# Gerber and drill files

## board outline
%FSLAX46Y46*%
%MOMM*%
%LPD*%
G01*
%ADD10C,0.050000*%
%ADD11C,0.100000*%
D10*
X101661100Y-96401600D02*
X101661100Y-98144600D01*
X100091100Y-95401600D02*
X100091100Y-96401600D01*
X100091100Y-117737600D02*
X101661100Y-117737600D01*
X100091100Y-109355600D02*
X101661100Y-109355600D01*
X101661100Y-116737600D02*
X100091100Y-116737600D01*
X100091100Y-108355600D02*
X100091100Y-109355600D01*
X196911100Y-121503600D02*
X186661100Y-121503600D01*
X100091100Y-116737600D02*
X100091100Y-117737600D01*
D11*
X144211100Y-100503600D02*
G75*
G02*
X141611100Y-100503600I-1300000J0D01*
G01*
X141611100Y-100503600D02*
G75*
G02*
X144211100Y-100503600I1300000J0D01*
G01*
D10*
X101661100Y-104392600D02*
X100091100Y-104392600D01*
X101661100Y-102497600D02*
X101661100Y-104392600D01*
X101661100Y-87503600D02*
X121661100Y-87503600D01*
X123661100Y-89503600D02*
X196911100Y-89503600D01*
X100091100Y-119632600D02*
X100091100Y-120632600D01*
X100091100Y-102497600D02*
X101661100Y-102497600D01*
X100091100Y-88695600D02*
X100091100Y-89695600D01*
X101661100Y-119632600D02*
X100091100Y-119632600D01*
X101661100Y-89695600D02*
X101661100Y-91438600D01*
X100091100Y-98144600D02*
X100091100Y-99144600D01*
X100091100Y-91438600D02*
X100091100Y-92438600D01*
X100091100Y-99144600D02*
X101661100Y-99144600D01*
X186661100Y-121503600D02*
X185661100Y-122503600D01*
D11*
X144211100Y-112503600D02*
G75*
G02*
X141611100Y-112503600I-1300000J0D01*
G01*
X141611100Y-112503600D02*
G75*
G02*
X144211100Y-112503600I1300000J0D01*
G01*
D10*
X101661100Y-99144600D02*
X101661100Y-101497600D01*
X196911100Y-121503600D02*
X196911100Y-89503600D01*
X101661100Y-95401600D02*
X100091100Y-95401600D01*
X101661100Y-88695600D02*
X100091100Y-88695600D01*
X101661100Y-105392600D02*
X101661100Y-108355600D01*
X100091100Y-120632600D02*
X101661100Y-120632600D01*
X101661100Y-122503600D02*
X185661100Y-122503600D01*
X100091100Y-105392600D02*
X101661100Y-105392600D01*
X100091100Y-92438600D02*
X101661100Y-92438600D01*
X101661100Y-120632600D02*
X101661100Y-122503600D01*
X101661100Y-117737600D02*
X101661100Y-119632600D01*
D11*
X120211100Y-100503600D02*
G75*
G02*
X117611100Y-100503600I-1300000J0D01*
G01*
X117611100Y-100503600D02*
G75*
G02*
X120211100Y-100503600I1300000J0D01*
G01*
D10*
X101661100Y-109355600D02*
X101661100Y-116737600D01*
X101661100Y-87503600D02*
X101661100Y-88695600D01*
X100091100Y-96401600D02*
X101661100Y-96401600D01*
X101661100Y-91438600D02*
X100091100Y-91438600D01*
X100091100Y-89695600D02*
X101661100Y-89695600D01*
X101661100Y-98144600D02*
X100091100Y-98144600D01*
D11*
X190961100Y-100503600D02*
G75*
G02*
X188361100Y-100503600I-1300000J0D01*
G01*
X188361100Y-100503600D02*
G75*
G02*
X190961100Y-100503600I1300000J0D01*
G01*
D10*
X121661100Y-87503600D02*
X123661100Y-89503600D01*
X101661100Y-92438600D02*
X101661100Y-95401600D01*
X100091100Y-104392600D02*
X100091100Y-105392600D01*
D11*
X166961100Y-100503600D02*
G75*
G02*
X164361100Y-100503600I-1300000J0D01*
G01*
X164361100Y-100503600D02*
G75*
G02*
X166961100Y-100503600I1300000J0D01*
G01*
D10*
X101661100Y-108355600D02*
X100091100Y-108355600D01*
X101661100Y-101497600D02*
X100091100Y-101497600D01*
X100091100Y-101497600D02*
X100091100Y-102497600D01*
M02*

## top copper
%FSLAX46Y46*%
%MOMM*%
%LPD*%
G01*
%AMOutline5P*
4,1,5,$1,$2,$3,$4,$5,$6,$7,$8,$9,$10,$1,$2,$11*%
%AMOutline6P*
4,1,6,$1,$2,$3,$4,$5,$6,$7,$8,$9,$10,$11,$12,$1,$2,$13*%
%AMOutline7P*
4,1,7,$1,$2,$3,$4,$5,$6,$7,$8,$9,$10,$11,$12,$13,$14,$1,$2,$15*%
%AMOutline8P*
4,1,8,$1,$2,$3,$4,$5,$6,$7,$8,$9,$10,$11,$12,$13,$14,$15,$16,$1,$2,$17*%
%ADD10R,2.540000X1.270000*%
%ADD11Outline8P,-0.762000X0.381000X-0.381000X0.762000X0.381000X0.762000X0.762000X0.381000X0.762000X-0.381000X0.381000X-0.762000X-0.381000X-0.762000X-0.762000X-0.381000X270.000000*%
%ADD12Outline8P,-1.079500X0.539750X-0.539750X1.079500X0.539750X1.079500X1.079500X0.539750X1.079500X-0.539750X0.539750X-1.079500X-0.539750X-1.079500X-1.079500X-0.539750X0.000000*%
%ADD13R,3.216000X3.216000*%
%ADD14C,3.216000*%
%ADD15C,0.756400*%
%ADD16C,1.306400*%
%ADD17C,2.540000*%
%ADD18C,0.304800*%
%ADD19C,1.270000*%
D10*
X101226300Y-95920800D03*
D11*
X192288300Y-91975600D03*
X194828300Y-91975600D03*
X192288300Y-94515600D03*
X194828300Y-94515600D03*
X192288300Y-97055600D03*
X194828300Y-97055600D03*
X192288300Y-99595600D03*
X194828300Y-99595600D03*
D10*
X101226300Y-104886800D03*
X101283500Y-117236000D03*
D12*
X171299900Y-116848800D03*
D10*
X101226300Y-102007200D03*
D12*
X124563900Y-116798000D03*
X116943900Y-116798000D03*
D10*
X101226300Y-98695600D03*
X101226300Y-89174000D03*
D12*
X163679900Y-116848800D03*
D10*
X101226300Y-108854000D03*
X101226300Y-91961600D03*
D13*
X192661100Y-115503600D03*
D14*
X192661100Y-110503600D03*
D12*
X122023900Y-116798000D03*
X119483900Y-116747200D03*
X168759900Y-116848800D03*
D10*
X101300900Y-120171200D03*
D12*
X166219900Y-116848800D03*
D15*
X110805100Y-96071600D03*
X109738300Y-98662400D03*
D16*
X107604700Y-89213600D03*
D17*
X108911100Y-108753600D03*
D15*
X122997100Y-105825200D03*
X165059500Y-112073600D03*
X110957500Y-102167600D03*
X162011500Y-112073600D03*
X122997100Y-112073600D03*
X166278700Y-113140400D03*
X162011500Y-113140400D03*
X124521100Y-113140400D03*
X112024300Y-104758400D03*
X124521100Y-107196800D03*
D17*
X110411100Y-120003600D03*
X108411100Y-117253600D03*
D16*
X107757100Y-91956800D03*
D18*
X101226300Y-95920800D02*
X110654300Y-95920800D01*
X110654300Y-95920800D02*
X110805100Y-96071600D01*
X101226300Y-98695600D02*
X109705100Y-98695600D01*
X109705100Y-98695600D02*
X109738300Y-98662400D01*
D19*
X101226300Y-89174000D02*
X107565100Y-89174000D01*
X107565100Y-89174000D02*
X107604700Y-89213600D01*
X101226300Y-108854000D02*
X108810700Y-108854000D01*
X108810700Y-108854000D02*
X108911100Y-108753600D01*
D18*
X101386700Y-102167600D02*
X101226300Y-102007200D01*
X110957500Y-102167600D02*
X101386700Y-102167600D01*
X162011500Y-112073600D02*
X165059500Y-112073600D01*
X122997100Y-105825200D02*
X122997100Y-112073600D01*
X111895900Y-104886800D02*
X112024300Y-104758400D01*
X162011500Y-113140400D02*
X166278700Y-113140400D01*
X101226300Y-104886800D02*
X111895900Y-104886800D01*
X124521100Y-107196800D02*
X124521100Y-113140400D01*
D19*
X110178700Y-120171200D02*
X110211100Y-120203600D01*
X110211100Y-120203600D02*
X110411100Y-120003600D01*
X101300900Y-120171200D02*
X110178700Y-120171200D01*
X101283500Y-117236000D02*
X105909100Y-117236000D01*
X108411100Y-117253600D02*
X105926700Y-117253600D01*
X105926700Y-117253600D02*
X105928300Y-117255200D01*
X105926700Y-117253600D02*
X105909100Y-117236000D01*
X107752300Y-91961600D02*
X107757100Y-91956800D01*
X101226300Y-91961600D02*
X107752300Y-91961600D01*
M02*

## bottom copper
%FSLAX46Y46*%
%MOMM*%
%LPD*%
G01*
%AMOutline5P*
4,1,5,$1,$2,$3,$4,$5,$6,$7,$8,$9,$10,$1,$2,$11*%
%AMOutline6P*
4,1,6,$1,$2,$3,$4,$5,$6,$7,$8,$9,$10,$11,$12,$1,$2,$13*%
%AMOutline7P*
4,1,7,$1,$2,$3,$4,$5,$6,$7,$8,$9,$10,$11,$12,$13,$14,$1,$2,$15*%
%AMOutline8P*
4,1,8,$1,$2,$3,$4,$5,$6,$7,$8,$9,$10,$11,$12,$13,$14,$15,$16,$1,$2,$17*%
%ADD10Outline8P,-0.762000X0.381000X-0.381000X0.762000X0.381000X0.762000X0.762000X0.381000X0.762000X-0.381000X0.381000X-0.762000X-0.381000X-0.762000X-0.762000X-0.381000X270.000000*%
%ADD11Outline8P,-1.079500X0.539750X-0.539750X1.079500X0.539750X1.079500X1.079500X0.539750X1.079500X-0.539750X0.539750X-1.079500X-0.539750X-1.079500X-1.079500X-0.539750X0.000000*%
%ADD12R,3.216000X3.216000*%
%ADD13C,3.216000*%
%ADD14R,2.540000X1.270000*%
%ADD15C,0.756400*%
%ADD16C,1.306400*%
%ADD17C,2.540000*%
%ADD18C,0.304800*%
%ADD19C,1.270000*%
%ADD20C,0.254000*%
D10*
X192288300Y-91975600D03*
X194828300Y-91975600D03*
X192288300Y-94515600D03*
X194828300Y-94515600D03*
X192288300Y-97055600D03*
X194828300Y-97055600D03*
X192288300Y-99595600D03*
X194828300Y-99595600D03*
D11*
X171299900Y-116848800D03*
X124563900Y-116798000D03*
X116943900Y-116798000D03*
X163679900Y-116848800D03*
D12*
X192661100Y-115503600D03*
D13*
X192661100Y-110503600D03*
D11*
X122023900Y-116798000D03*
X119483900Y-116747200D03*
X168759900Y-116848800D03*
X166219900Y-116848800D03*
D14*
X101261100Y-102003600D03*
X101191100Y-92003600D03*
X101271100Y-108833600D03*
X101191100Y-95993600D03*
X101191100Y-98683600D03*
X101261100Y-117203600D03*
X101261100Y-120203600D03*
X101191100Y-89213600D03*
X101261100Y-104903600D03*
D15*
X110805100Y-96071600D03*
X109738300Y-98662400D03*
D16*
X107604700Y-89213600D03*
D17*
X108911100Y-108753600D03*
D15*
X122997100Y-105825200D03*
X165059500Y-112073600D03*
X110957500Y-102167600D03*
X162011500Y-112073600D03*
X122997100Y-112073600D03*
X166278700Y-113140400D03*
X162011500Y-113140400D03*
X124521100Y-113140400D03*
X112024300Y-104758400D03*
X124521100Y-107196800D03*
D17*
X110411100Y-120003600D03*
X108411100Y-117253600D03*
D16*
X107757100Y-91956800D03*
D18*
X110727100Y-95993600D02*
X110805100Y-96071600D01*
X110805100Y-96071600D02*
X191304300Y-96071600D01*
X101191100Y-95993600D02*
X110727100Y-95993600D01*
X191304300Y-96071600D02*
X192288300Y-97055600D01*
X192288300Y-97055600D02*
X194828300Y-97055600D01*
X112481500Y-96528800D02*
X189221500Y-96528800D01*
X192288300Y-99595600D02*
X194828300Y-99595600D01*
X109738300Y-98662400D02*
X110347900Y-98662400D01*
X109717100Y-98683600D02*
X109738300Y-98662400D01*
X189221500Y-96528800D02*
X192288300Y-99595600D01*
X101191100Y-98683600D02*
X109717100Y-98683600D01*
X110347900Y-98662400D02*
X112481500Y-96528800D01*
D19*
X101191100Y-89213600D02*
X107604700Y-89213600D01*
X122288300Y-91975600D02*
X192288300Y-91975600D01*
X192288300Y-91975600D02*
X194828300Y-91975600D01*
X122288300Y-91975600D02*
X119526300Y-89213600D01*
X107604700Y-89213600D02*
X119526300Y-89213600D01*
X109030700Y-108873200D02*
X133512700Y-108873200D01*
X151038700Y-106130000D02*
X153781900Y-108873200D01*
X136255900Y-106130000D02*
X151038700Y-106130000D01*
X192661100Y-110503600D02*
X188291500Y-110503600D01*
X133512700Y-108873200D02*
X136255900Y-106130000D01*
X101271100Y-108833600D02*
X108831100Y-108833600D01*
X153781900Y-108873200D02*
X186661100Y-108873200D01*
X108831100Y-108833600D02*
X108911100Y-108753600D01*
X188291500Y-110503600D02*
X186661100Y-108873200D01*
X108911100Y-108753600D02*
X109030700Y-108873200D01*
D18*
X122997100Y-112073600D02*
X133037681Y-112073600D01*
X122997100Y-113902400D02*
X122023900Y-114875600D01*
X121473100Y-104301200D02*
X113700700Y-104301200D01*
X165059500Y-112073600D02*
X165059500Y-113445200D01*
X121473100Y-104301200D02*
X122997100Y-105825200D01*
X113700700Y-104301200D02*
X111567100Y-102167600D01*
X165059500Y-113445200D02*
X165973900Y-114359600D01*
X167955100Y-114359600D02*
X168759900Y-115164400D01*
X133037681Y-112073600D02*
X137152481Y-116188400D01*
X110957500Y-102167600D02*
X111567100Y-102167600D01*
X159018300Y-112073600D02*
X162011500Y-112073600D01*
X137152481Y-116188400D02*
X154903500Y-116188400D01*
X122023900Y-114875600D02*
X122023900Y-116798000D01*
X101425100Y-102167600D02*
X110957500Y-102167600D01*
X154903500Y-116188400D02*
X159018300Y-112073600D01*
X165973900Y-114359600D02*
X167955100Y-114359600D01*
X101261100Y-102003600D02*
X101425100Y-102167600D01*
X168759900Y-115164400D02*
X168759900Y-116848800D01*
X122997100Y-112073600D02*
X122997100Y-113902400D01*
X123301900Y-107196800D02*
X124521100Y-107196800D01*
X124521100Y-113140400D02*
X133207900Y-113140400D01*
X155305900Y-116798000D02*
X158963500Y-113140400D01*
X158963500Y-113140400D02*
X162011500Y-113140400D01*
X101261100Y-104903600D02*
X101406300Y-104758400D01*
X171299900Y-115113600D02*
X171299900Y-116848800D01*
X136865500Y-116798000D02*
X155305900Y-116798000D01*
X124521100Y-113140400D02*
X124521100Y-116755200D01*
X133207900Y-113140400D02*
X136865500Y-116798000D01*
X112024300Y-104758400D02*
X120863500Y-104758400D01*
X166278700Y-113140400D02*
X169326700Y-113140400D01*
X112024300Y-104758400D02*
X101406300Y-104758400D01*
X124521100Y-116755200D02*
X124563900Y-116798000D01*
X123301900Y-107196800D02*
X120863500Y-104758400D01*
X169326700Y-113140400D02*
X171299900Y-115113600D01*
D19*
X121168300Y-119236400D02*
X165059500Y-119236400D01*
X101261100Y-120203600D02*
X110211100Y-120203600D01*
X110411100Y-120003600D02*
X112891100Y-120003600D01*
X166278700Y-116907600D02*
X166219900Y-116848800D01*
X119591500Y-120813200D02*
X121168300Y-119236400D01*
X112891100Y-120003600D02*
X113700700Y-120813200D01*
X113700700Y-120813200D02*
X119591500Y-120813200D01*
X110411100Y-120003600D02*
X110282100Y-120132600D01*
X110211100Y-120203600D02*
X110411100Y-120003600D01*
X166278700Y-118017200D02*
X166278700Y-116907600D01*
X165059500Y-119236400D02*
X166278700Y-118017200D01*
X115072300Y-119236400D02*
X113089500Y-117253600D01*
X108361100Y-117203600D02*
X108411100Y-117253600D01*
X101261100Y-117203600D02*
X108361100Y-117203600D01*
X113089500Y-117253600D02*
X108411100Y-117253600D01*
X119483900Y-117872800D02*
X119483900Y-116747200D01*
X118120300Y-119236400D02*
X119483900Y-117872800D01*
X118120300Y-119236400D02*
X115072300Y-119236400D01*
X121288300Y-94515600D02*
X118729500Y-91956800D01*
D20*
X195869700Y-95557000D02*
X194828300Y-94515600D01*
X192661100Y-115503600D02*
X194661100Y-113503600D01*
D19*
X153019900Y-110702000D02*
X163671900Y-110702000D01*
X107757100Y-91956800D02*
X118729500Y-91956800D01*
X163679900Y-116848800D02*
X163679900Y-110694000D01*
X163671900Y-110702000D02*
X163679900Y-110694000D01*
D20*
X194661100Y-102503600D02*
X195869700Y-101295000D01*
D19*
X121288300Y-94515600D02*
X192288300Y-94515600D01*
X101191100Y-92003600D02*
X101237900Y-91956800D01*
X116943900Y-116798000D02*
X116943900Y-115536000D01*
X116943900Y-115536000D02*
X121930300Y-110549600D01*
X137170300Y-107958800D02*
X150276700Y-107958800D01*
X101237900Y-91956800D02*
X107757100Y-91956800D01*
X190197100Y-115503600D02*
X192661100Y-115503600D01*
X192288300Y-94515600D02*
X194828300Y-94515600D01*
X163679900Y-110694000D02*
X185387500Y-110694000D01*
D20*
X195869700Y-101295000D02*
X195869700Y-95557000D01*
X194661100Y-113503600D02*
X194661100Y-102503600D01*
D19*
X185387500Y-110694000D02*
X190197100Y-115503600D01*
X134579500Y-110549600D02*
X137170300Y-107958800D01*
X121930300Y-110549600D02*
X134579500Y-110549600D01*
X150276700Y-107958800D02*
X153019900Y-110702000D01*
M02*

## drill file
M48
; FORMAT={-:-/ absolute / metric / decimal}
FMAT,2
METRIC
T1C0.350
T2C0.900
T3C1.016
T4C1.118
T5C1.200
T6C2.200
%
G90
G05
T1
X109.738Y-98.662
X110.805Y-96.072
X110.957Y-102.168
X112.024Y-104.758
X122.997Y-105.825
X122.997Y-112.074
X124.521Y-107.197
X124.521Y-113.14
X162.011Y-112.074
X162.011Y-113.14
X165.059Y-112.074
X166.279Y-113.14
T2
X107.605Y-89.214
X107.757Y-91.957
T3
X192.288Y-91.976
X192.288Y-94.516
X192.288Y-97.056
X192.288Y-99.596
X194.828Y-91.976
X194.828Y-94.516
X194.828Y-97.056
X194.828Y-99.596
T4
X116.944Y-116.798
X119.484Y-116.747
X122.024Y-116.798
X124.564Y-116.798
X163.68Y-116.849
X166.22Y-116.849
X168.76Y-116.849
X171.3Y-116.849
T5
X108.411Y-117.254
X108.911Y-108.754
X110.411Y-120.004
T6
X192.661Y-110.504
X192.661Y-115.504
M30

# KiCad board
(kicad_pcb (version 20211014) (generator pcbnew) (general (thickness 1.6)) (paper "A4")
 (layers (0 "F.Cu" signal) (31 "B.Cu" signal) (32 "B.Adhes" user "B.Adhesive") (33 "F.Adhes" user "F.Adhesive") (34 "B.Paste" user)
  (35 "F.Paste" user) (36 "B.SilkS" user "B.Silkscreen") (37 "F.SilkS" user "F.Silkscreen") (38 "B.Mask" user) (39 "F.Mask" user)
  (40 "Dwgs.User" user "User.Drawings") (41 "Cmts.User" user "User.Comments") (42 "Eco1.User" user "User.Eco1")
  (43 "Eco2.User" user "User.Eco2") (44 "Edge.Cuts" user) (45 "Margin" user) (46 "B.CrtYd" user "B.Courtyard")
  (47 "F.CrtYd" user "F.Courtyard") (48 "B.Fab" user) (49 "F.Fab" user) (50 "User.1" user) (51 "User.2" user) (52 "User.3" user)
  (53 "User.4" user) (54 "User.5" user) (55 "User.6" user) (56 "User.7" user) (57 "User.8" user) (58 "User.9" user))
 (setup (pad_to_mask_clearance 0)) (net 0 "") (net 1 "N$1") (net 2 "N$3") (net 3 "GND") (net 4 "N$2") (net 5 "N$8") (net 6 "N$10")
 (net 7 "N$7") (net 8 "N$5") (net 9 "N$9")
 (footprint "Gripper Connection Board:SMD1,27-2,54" (layer "F.Cu") (at 101.2263 95.9208 90)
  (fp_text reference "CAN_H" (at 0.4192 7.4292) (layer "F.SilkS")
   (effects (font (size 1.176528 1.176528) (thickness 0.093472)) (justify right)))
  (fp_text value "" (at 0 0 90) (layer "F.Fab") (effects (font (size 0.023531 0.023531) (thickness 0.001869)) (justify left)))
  (pad "1" smd rect (at 0 0 90) (size 1.27 2.54) (layers "F.Cu" "F.Paste" "F.Mask") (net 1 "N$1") (solder_mask_margin 0.1016)))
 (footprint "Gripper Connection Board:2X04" (layer "F.Cu") (at 193.5583 95.7856 -90)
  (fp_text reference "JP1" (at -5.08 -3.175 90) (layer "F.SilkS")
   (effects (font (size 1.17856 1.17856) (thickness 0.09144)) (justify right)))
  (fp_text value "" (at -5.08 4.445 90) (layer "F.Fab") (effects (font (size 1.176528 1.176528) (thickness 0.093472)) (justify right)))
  (pad "1" thru_hole roundrect (at -3.81 1.27 270) (size 1.524 1.524) (drill 1.016) (layers *.Cu *.Mask) (roundrect_rratio 0.25)
   (chamfer_ratio 0.25) (chamfer top_left top_right bottom_left bottom_right) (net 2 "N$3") (solder_mask_margin 0.1016))
  (pad "2" thru_hole roundrect (at -3.81 -1.27 270) (size 1.524 1.524) (drill 1.016) (layers *.Cu *.Mask) (roundrect_rratio 0.25)
   (chamfer_ratio 0.25) (chamfer top_left top_right bottom_left bottom_right) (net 2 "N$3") (solder_mask_margin 0.1016))
  (pad "3" thru_hole roundrect (at -1.27 1.27 270) (size 1.524 1.524) (drill 1.016) (layers *.Cu *.Mask) (roundrect_rratio 0.25)
   (chamfer_ratio 0.25) (chamfer top_left top_right bottom_left bottom_right) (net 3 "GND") (solder_mask_margin 0.1016))
  (pad "4" thru_hole roundrect (at -1.27 -1.27 270) (size 1.524 1.524) (drill 1.016) (layers *.Cu *.Mask) (roundrect_rratio 0.25)
   (chamfer_ratio 0.25) (chamfer top_left top_right bottom_left bottom_right) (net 3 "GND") (solder_mask_margin 0.1016))
  (pad "5" thru_hole roundrect (at 1.27 1.27 270) (size 1.524 1.524) (drill 1.016) (layers *.Cu *.Mask) (roundrect_rratio 0.25)
   (chamfer_ratio 0.25) (chamfer top_left top_right bottom_left bottom_right) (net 1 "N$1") (solder_mask_margin 0.1016))
  (pad "6" thru_hole roundrect (at 1.27 -1.27 270) (size 1.524 1.524) (drill 1.016) (layers *.Cu *.Mask) (roundrect_rratio 0.25)
   (chamfer_ratio 0.25) (chamfer top_left top_right bottom_left bottom_right) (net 1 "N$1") (solder_mask_margin 0.1016))
  (pad "7" thru_hole roundrect (at 3.81 1.27 270) (size 1.524 1.524) (drill 1.016) (layers *.Cu *.Mask) (roundrect_rratio 0.25)
   (chamfer_ratio 0.25) (chamfer top_left top_right bottom_left bottom_right) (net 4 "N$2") (solder_mask_margin 0.1016))
  (pad "8" thru_hole roundrect (at 3.81 -1.27 270) (size 1.524 1.524) (drill 1.016) (layers *.Cu *.Mask) (roundrect_rratio 0.25)
   (chamfer_ratio 0.25) (chamfer top_left top_right bottom_left bottom_right) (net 4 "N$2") (solder_mask_margin 0.1016)))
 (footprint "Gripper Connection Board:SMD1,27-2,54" (layer "F.Cu") (at 101.2263 104.8868 90)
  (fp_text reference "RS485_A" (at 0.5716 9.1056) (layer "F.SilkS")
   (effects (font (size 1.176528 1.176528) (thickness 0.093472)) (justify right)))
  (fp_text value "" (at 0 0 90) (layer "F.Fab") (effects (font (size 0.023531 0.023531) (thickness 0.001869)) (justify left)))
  (pad "1" smd rect (at 0 0 90) (size 1.27 2.54) (layers "F.Cu" "F.Paste" "F.Mask") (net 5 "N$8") (solder_mask_margin 0.1016)))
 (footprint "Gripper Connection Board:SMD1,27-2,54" (layer "F.Cu") (at 101.2835 117.236 90)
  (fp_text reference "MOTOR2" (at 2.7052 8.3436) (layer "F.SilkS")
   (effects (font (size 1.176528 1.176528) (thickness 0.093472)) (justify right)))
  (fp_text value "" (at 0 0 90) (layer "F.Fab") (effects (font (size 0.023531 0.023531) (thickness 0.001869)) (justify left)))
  (pad "1" smd rect (at 0 0 90) (size 1.27 2.54) (layers "F.Cu" "F.Paste" "F.Mask") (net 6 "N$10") (solder_mask_margin 0.1016)))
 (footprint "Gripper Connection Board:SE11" (layer "F.Cu") (at 171.2999 116.8488)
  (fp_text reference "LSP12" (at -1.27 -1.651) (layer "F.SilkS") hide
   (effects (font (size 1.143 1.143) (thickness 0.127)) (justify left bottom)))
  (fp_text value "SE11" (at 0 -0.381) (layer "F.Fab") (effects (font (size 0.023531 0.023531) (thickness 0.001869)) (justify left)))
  (pad "MP" thru_hole roundrect (at 0 0) (size 2.159 2.159) (drill 1.1176) (layers *.Cu *.Mask) (roundrect_rratio 0.25) (chamfer_ratio 0.25)
   (chamfer top_left top_right bottom_left bottom_right) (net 5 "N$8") (solder_mask_margin 0.1016)))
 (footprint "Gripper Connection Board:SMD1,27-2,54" (layer "F.Cu") (at 101.2263 102.0072 90)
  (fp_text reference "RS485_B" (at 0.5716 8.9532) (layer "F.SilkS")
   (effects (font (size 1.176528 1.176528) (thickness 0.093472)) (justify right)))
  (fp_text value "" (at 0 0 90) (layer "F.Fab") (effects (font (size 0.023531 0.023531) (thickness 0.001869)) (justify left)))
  (pad "1" smd rect (at 0 0 90) (size 1.27 2.54) (layers "F.Cu" "F.Paste" "F.Mask") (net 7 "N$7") (solder_mask_margin 0.1016)))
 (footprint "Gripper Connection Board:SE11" (layer "F.Cu") (at 124.5639 116.798)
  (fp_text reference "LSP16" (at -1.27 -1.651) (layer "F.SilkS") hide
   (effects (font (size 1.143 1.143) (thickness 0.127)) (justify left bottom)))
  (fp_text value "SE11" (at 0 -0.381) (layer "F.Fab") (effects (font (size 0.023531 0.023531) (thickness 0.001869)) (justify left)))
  (pad "MP" thru_hole roundrect (at 0 0) (size 2.159 2.159) (drill 1.1176) (layers *.Cu *.Mask) (roundrect_rratio 0.25) (chamfer_ratio 0.25)
   (chamfer top_left top_right bottom_left bottom_right) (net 5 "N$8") (solder_mask_margin 0.1016)))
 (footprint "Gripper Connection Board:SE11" (layer "F.Cu") (at 116.9439 116.798)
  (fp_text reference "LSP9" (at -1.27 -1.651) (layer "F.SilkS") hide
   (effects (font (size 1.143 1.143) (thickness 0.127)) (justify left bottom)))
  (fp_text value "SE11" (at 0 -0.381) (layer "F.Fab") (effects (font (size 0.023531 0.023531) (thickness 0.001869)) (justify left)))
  (pad "MP" thru_hole roundrect (at 0 0) (size 2.159 2.159) (drill 1.1176) (layers *.Cu *.Mask) (roundrect_rratio 0.25) (chamfer_ratio 0.25)
   (chamfer top_left top_right bottom_left bottom_right) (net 3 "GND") (solder_mask_margin 0.1016)))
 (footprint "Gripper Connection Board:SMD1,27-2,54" (layer "F.Cu") (at 101.2263 98.6956 90)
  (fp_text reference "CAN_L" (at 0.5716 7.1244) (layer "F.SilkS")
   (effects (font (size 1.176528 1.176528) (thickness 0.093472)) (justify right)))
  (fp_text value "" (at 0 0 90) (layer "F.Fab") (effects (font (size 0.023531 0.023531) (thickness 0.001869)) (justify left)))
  (pad "1" smd rect (at 0 0 90) (size 1.27 2.54) (layers "F.Cu" "F.Paste" "F.Mask") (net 4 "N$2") (solder_mask_margin 0.1016)))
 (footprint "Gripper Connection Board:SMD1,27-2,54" (layer "F.Cu") (at 101.2263 89.174 90)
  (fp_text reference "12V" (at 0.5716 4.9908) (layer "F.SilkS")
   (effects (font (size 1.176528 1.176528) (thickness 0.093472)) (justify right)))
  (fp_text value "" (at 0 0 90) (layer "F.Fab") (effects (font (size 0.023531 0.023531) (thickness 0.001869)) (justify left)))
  (pad "1" smd rect (at 0 0 90) (size 1.27 2.54) (layers "F.Cu" "F.Paste" "F.Mask") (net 2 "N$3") (solder_mask_margin 0.1016)))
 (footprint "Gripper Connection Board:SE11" (layer "F.Cu") (at 163.6799 116.8488)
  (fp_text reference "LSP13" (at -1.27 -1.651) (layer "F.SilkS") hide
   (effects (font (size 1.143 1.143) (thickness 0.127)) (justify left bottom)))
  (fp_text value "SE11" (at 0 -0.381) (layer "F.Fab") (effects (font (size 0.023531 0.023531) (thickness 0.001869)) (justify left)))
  (pad "MP" thru_hole roundrect (at 0 0) (size 2.159 2.159) (drill 1.1176) (layers *.Cu *.Mask) (roundrect_rratio 0.25) (chamfer_ratio 0.25)
   (chamfer top_left top_right bottom_left bottom_right) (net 3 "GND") (solder_mask_margin 0.1016)))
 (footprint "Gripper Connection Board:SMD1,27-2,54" (layer "F.Cu") (at 101.2263 108.854 90)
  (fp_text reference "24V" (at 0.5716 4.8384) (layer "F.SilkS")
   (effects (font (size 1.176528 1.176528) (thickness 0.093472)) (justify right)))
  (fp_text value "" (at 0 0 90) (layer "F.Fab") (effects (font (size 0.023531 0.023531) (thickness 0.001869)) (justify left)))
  (pad "1" smd rect (at 0 0 90) (size 1.27 2.54) (layers "F.Cu" "F.Paste" "F.Mask") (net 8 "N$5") (solder_mask_margin 0.1016)))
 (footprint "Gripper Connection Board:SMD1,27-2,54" (layer "F.Cu") (at 101.2263 91.9616 90)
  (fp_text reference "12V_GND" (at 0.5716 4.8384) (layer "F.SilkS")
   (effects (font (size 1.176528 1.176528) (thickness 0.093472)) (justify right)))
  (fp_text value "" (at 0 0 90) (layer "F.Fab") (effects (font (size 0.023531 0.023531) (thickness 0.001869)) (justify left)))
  (pad "1" smd rect (at 0 0 90) (size 1.27 2.54) (layers "F.Cu" "F.Paste" "F.Mask") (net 3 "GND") (solder_mask_margin 0.1016)))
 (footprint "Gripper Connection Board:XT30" (layer "F.Cu") (at 192.6611 113.5036 90)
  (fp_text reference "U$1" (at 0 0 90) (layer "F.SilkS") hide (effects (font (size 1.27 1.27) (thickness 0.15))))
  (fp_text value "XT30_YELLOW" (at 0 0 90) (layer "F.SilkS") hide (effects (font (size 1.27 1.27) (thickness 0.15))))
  (pad "P$1" thru_hole rect (at -2 0 90) (size 3.216 3.216) (drill 2.2) (layers *.Cu *.Mask) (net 3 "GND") (solder_mask_margin 0.1016))
  (pad "P$2" thru_hole circle (at 3 0 90) (size 3.216 3.216) (drill 2.2) (layers *.Cu *.Mask) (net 8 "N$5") (solder_mask_margin 0.1016)))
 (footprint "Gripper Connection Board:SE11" (layer "F.Cu") (at 122.0239 116.798)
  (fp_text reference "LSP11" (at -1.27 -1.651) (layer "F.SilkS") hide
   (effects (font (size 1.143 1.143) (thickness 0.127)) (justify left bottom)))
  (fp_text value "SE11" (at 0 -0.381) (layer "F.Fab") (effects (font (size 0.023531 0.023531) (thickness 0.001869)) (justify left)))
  (pad "MP" thru_hole roundrect (at 0 0) (size 2.159 2.159) (drill 1.1176) (layers *.Cu *.Mask) (roundrect_rratio 0.25) (chamfer_ratio 0.25)
   (chamfer top_left top_right bottom_left bottom_right) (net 7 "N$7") (solder_mask_margin 0.1016)))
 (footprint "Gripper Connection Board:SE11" (layer "F.Cu") (at 119.4839 116.7472)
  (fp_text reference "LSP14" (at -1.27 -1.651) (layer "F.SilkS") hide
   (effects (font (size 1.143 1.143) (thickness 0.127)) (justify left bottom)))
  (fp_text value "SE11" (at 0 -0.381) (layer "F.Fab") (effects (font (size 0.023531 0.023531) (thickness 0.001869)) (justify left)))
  (pad "MP" thru_hole roundrect (at 0 0) (size 2.159 2.159) (drill 1.1176) (layers *.Cu *.Mask) (roundrect_rratio 0.25) (chamfer_ratio 0.25)
   (chamfer top_left top_right bottom_left bottom_right) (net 6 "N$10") (solder_mask_margin 0.1016)))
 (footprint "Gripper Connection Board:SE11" (layer "F.Cu") (at 168.7599 116.8488)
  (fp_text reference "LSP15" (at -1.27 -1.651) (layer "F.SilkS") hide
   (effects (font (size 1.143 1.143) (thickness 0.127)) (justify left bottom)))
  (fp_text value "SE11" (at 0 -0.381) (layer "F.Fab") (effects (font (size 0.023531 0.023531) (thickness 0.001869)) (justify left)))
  (pad "MP" thru_hole roundrect (at 0 0) (size 2.159 2.159) (drill 1.1176) (layers *.Cu *.Mask) (roundrect_rratio 0.25) (chamfer_ratio 0.25)
   (chamfer top_left top_right bottom_left bottom_right) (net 7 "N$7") (solder_mask_margin 0.1016)))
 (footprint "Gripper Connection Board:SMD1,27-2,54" (layer "F.Cu") (at 101.3009 120.1712 90)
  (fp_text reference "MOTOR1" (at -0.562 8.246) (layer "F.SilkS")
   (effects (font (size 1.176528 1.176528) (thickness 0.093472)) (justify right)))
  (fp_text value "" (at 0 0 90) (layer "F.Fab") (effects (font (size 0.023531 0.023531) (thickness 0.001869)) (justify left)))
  (pad "1" smd rect (at 0 0 90) (size 1.27 2.54) (layers "F.Cu" "F.Paste" "F.Mask") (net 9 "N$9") (solder_mask_margin 0.1016)))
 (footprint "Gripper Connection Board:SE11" (layer "F.Cu") (at 166.2199 116.8488)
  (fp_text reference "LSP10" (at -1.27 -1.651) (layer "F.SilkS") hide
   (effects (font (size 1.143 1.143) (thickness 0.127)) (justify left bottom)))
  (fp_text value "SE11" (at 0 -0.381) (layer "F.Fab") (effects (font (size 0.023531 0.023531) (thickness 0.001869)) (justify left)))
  (pad "MP" thru_hole roundrect (at 0 0) (size 2.159 2.159) (drill 1.1176) (layers *.Cu *.Mask) (roundrect_rratio 0.25) (chamfer_ratio 0.25)
   (chamfer top_left top_right bottom_left bottom_right) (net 9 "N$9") (solder_mask_margin 0.1016)))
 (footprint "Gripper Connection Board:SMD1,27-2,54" (layer "B.Cu") (at 101.2611 102.0036 -90)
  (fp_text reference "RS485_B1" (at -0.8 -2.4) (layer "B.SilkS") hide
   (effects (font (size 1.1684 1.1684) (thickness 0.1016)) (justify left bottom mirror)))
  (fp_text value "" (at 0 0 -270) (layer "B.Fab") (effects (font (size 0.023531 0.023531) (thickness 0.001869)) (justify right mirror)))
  (pad "1" smd rect (at 0 0 270) (size 1.27 2.54) (layers "B.Cu" "B.Paste" "B.Mask") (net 7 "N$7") (solder_mask_margin 0.1016)))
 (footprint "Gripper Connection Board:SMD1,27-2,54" (layer "B.Cu") (at 101.1911 92.0036 -90)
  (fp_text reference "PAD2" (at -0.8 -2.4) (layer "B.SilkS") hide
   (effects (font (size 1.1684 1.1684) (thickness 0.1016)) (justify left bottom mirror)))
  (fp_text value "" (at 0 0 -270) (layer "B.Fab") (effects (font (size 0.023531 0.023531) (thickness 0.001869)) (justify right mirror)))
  (pad "1" smd rect (at 0 0 270) (size 1.27 2.54) (layers "B.Cu" "B.Paste" "B.Mask") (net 3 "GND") (solder_mask_margin 0.1016)))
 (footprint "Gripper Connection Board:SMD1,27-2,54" (layer "B.Cu") (at 101.2711 108.8336 -90)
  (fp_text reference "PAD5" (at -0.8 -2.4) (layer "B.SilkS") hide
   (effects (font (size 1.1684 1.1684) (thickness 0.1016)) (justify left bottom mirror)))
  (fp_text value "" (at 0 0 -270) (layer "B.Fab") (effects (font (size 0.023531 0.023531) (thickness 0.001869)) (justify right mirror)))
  (pad "1" smd rect (at 0 0 270) (size 1.27 2.54) (layers "B.Cu" "B.Paste" "B.Mask") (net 8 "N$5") (solder_mask_margin 0.1016)))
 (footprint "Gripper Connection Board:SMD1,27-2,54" (layer "B.Cu") (at 101.1911 95.9936 -90)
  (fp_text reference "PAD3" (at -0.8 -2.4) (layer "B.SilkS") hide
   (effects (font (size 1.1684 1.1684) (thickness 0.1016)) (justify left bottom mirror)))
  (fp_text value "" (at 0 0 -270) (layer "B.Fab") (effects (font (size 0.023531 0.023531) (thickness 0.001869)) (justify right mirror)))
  (pad "1" smd rect (at 0 0 270) (size 1.27 2.54) (layers "B.Cu" "B.Paste" "B.Mask") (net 1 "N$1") (solder_mask_margin 0.1016)))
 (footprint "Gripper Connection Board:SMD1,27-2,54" (layer "B.Cu") (at 101.1911 98.6836 -90)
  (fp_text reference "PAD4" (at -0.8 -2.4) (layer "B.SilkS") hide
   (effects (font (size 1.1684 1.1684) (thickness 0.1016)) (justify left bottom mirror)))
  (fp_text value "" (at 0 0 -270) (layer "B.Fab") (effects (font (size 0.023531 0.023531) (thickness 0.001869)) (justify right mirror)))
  (pad "1" smd rect (at 0 0 270) (size 1.27 2.54) (layers "B.Cu" "B.Paste" "B.Mask") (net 4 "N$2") (solder_mask_margin 0.1016)))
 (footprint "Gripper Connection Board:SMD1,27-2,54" (layer "B.Cu") (at 101.2611 117.2036 -90)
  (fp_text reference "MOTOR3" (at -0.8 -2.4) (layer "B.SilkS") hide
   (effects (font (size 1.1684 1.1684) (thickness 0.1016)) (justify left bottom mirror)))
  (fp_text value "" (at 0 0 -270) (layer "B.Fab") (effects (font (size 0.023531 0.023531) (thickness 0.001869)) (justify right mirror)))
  (pad "1" smd rect (at 0 0 270) (size 1.27 2.54) (layers "B.Cu" "B.Paste" "B.Mask") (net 6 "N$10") (solder_mask_margin 0.1016)))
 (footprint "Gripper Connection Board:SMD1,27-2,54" (layer "B.Cu") (at 101.2611 120.2036 -90)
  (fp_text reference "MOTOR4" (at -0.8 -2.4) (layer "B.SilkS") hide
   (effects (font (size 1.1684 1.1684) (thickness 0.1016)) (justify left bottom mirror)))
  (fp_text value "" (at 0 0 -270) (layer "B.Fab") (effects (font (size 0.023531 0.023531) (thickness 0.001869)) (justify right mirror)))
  (pad "1" smd rect (at 0 0 270) (size 1.27 2.54) (layers "B.Cu" "B.Paste" "B.Mask") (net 9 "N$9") (solder_mask_margin 0.1016)))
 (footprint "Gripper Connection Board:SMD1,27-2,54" (layer "B.Cu") (at 101.1911 89.2136 -90)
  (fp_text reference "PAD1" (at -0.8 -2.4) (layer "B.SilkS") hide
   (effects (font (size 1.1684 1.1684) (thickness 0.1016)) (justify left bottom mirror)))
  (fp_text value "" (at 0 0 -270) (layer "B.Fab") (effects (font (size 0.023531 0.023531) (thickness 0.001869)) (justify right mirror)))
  (pad "1" smd rect (at 0 0 270) (size 1.27 2.54) (layers "B.Cu" "B.Paste" "B.Mask") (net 2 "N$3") (solder_mask_margin 0.1016)))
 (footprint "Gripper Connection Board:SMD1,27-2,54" (layer "B.Cu") (at 101.2611 104.9036 -90)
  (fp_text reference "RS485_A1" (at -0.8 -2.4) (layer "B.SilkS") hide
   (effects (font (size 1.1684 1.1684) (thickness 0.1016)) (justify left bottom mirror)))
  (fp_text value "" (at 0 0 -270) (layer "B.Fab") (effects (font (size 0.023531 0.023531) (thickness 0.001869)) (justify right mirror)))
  (pad "1" smd rect (at 0 0 270) (size 1.27 2.54) (layers "B.Cu" "B.Paste" "B.Mask") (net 5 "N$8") (solder_mask_margin 0.1016)))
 (gr_line (start 101.6611 96.4016) (end 101.6611 98.1446) (layer "Edge.Cuts") (width 0.05))
 (gr_line (start 100.0911 95.4016) (end 100.0911 96.4016) (layer "Edge.Cuts") (width 0.05))
 (gr_line (start 100.0911 117.7376) (end 101.6611 117.7376) (layer "Edge.Cuts") (width 0.05))
 (gr_line (start 100.0911 109.3556) (end 101.6611 109.3556) (layer "Edge.Cuts") (width 0.05))
 (gr_line (start 101.6611 116.7376) (end 100.0911 116.7376) (layer "Edge.Cuts") (width 0.05))
 (gr_line (start 100.0911 108.3556) (end 100.0911 109.3556) (layer "Edge.Cuts") (width 0.05))
 (gr_line (start 196.9111 121.5036) (end 186.6611 121.5036) (layer "Edge.Cuts") (width 0.05))
 (gr_line (start 100.0911 116.7376) (end 100.0911 117.7376) (layer "Edge.Cuts") (width 0.05))
 (gr_circle (center 142.9111 100.5036) (end 144.2111 100.5036) (layer "Edge.Cuts") (width 0) (fill none))
 (gr_line (start 101.6611 104.3926) (end 100.0911 104.3926) (layer "Edge.Cuts") (width 0.05))
 (gr_line (start 101.6611 102.4976) (end 101.6611 104.3926) (layer "Edge.Cuts") (width 0.05))
 (gr_line (start 101.6611 87.5036) (end 121.6611 87.5036) (layer "Edge.Cuts") (width 0.05))
 (gr_line (start 123.6611 89.5036) (end 196.9111 89.5036) (layer "Edge.Cuts") (width 0.05))
 (gr_line (start 100.0911 119.6326) (end 100.0911 120.6326) (layer "Edge.Cuts") (width 0.05))
 (gr_line (start 100.0911 102.4976) (end 101.6611 102.4976) (layer "Edge.Cuts") (width 0.05))
 (gr_line (start 100.0911 88.6956) (end 100.0911 89.6956) (layer "Edge.Cuts") (width 0.05))
 (gr_line (start 101.6611 119.6326) (end 100.0911 119.6326) (layer "Edge.Cuts") (width 0.05))
 (gr_line (start 101.6611 89.6956) (end 101.6611 91.4386) (layer "Edge.Cuts") (width 0.05))
 (gr_line (start 100.0911 98.1446) (end 100.0911 99.1446) (layer "Edge.Cuts") (width 0.05))
 (gr_line (start 100.0911 91.4386) (end 100.0911 92.4386) (layer "Edge.Cuts") (width 0.05))
 (gr_line (start 100.0911 99.1446) (end 101.6611 99.1446) (layer "Edge.Cuts") (width 0.05))
 (gr_line (start 186.6611 121.5036) (end 185.6611 122.5036) (layer "Edge.Cuts") (width 0.05))
 (gr_circle (center 142.9111 112.5036) (end 144.2111 112.5036) (layer "Edge.Cuts") (width 0) (fill none))
 (gr_line (start 101.6611 99.1446) (end 101.6611 101.4976) (layer "Edge.Cuts") (width 0.05))
 (gr_line (start 196.9111 121.5036) (end 196.9111 89.5036) (layer "Edge.Cuts") (width 0.05))
 (gr_line (start 101.6611 95.4016) (end 100.0911 95.4016) (layer "Edge.Cuts") (width 0.05))
 (gr_line (start 101.6611 88.6956) (end 100.0911 88.6956) (layer "Edge.Cuts") (width 0.05))
 (gr_line (start 101.6611 105.3926) (end 101.6611 108.3556) (layer "Edge.Cuts") (width 0.05))
 (gr_line (start 100.0911 120.6326) (end 101.6611 120.6326) (layer "Edge.Cuts") (width 0.05))
 (gr_line (start 101.6611 122.5036) (end 185.6611 122.5036) (layer "Edge.Cuts") (width 0.05))
 (gr_line (start 100.0911 105.3926) (end 101.6611 105.3926) (layer "Edge.Cuts") (width 0.05))
 (gr_line (start 100.0911 92.4386) (end 101.6611 92.4386) (layer "Edge.Cuts") (width 0.05))
 (gr_line (start 101.6611 120.6326) (end 101.6611 122.5036) (layer "Edge.Cuts") (width 0.05))
 (gr_line (start 101.6611 117.7376) (end 101.6611 119.6326) (layer "Edge.Cuts") (width 0.05))
 (gr_circle (center 118.9111 100.5036) (end 120.2111 100.5036) (layer "Edge.Cuts") (width 0) (fill none))
 (gr_line (start 101.6611 109.3556) (end 101.6611 116.7376) (layer "Edge.Cuts") (width 0.05))
 (gr_line (start 101.6611 87.5036) (end 101.6611 88.6956) (layer "Edge.Cuts") (width 0.05))
 (gr_line (start 100.0911 96.4016) (end 101.6611 96.4016) (layer "Edge.Cuts") (width 0.05))
 (gr_line (start 101.6611 91.4386) (end 100.0911 91.4386) (layer "Edge.Cuts") (width 0.05))
 (gr_line (start 100.0911 89.6956) (end 101.6611 89.6956) (layer "Edge.Cuts") (width 0.05))
 (gr_line (start 101.6611 98.1446) (end 100.0911 98.1446) (layer "Edge.Cuts") (width 0.05))
 (gr_circle (center 189.6611 100.5036) (end 190.9611 100.5036) (layer "Edge.Cuts") (width 0) (fill none))
 (gr_line (start 121.6611 87.5036) (end 123.6611 89.5036) (layer "Edge.Cuts") (width 0.05))
 (gr_line (start 101.6611 92.4386) (end 101.6611 95.4016) (layer "Edge.Cuts") (width 0.05))
 (gr_line (start 100.0911 104.3926) (end 100.0911 105.3926) (layer "Edge.Cuts") (width 0.05))
 (gr_circle (center 165.6611 100.5036) (end 166.9611 100.5036) (layer "Edge.Cuts") (width 0) (fill none))
 (gr_line (start 101.6611 108.3556) (end 100.0911 108.3556) (layer "Edge.Cuts") (width 0.05))
 (gr_line (start 101.6611 101.4976) (end 100.0911 101.4976) (layer "Edge.Cuts") (width 0.05))
 (gr_line (start 100.0911 101.4976) (end 100.0911 102.4976) (layer "Edge.Cuts") (width 0.05))
 (segment (start 101.2263 95.9208) (end 110.6543 95.9208) (width 0.3048) (layer "F.Cu") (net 1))
 (segment (start 110.6543 95.9208) (end 110.8051 96.0716) (width 0.3048) (layer "F.Cu") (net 1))
 (via (at 110.8051 96.0716) (size 0.7564) (drill 0.35) (layers "F.Cu" "B.Cu") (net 1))
 (segment (start 110.7271 95.9936) (end 110.8051 96.0716) (width 0.3048) (layer "B.Cu") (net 1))
 (segment (start 110.8051 96.0716) (end 191.3043 96.0716) (width 0.3048) (layer "B.Cu") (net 1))
 (segment (start 101.1911 95.9936) (end 110.7271 95.9936) (width 0.3048) (layer "B.Cu") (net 1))
 (segment (start 191.3043 96.0716) (end 192.2883 97.0556) (width 0.3048) (layer "B.Cu") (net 1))
 (segment (start 192.2883 97.0556) (end 194.8283 97.0556) (width 0.3048) (layer "B.Cu") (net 1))
 (segment (start 101.2263 98.6956) (end 109.7051 98.6956) (width 0.3048) (layer "F.Cu") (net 4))
 (segment (start 109.7051 98.6956) (end 109.7383 98.6624) (width 0.3048) (layer "F.Cu") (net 4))
 (via (at 109.7383 98.6624) (size 0.7564) (drill 0.35) (layers "F.Cu" "B.Cu") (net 4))
 (segment (start 112.4815 96.5288) (end 189.2215 96.5288) (width 0.3048) (layer "B.Cu") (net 4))
 (segment (start 192.2883 99.5956) (end 194.8283 99.5956) (width 0.3048) (layer "B.Cu") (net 4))
 (segment (start 109.7383 98.6624) (end 110.3479 98.6624) (width 0.3048) (layer "B.Cu") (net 4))
 (segment (start 109.7171 98.6836) (end 109.7383 98.6624) (width 0.3048) (layer "B.Cu") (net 4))
 (segment (start 189.2215 96.5288) (end 192.2883 99.5956) (width 0.3048) (layer "B.Cu") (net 4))
 (segment (start 101.1911 98.6836) (end 109.7171 98.6836) (width 0.3048) (layer "B.Cu") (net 4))
 (segment (start 110.3479 98.6624) (end 112.4815 96.5288) (width 0.3048) (layer "B.Cu") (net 4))
 (segment (start 101.2263 89.174) (end 107.5651 89.174) (width 1.27) (layer "F.Cu") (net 2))
 (segment (start 107.5651 89.174) (end 107.6047 89.2136) (width 1.27) (layer "F.Cu") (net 2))
 (via (at 107.6047 89.2136) (size 1.3064) (drill 0.9) (layers "F.Cu" "B.Cu") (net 2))
 (segment (start 101.1911 89.2136) (end 107.6047 89.2136) (width 1.27) (layer "B.Cu") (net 2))
 (segment (start 122.2883 91.9756) (end 192.2883 91.9756) (width 1.27) (layer "B.Cu") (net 2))
 (segment (start 192.2883 91.9756) (end 194.8283 91.9756) (width 1.27) (layer "B.Cu") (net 2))
 (segment (start 122.2883 91.9756) (end 119.5263 89.2136) (width 1.27) (layer "B.Cu") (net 2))
 (segment (start 107.6047 89.2136) (end 119.5263 89.2136) (width 1.27) (layer "B.Cu") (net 2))
 (segment (start 101.2263 108.854) (end 108.8107 108.854) (width 1.27) (layer "F.Cu") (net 8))
 (segment (start 108.8107 108.854) (end 108.9111 108.7536) (width 1.27) (layer "F.Cu") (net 8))
 (via (at 108.9111 108.7536) (size 2.54) (drill 1.2) (layers "F.Cu" "B.Cu") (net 8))
 (segment (start 109.0307 108.8732) (end 133.5127 108.8732) (width 1.27) (layer "B.Cu") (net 8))
 (segment (start 151.0387 106.13) (end 153.7819 108.8732) (width 1.27) (layer "B.Cu") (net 8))
 (segment (start 136.2559 106.13) (end 151.0387 106.13) (width 1.27) (layer "B.Cu") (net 8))
 (segment (start 192.6611 110.5036) (end 188.2915 110.5036) (width 1.27) (layer "B.Cu") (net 8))
 (segment (start 133.5127 108.8732) (end 136.2559 106.13) (width 1.27) (layer "B.Cu") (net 8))
 (segment (start 101.2711 108.8336) (end 108.8311 108.8336) (width 1.27) (layer "B.Cu") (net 8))
 (segment (start 153.7819 108.8732) (end 186.6611 108.8732) (width 1.27) (layer "B.Cu") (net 8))
 (segment (start 108.8311 108.8336) (end 108.9111 108.7536) (width 1.27) (layer "B.Cu") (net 8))
 (segment (start 188.2915 110.5036) (end 186.6611 108.8732) (width 1.27) (layer "B.Cu") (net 8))
 (segment (start 108.9111 108.7536) (end 109.0307 108.8732) (width 1.27) (layer "B.Cu") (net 8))
 (segment (start 101.3867 102.1676) (end 101.2263 102.0072) (width 0.3048) (layer "F.Cu") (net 7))
 (segment (start 110.9575 102.1676) (end 101.3867 102.1676) (width 0.3048) (layer "F.Cu") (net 7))
 (segment (start 162.0115 112.0736) (end 165.0595 112.0736) (width 0.3048) (layer "F.Cu") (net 7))
 (segment (start 122.9971 105.8252) (end 122.9971 112.0736) (width 0.3048) (layer "F.Cu") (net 7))
 (via (at 122.9971 105.8252) (size 0.7564) (drill 0.35) (layers "F.Cu" "B.Cu") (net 7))
 (via (at 165.0595 112.0736) (size 0.7564) (drill 0.35) (layers "F.Cu" "B.Cu") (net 7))
 (via (at 110.9575 102.1676) (size 0.7564) (drill 0.35) (layers "F.Cu" "B.Cu") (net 7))
 (via (at 162.0115 112.0736) (size 0.7564) (drill 0.35) (layers "F.Cu" "B.Cu") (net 7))
 (via (at 122.9971 112.0736) (size 0.7564) (drill 0.35) (layers "F.Cu" "B.Cu") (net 7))
 (segment (start 122.9971 112.0736) (end 133.037681 112.0736) (width 0.3048) (layer "B.Cu") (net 7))
 (segment (start 122.9971 113.9024) (end 122.0239 114.8756) (width 0.3048) (layer "B.Cu") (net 7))
 (segment (start 121.4731 104.3012) (end 113.7007 104.3012) (width 0.3048) (layer "B.Cu") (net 7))
 (segment (start 165.0595 112.0736) (end 165.0595 113.4452) (width 0.3048) (layer "B.Cu") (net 7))
 (segment (start 121.4731 104.3012) (end 122.9971 105.8252) (width 0.3048) (layer "B.Cu") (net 7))
 (segment (start 113.7007 104.3012) (end 111.5671 102.1676) (width 0.3048) (layer "B.Cu") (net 7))
 (segment (start 165.0595 113.4452) (end 165.9739 114.3596) (width 0.3048) (layer "B.Cu") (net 7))
 (segment (start 167.9551 114.3596) (end 168.7599 115.1644) (width 0.3048) (layer "B.Cu") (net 7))
 (segment (start 133.037681 112.0736) (end 137.152481 116.1884) (width 0.3048) (layer "B.Cu") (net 7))
 (segment (start 110.9575 102.1676) (end 111.5671 102.1676) (width 0.3048) (layer "B.Cu") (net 7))
 (segment (start 159.0183 112.0736) (end 162.0115 112.0736) (width 0.3048) (layer "B.Cu") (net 7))
 (segment (start 137.152481 116.1884) (end 154.9035 116.1884) (width 0.3048) (layer "B.Cu") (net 7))
 (segment (start 122.0239 114.8756) (end 122.0239 116.798) (width 0.3048) (layer "B.Cu") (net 7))
 (segment (start 101.4251 102.1676) (end 110.9575 102.1676) (width 0.3048) (layer "B.Cu") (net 7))
 (segment (start 154.9035 116.1884) (end 159.0183 112.0736) (width 0.3048) (layer "B.Cu") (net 7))
 (segment (start 165.9739 114.3596) (end 167.9551 114.3596) (width 0.3048) (layer "B.Cu") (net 7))
 (segment (start 101.2611 102.0036) (end 101.4251 102.1676) (width 0.3048) (layer "B.Cu") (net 7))
 (segment (start 168.7599 115.1644) (end 168.7599 116.8488) (width 0.3048) (layer "B.Cu") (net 7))
 (segment (start 122.9971 112.0736) (end 122.9971 113.9024) (width 0.3048) (layer "B.Cu") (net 7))
 (segment (start 111.8959 104.8868) (end 112.0243 104.7584) (width 0.3048) (layer "F.Cu") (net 5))
 (segment (start 162.0115 113.1404) (end 166.2787 113.1404) (width 0.3048) (layer "F.Cu") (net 5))
 (segment (start 101.2263 104.8868) (end 111.8959 104.8868) (width 0.3048) (layer "F.Cu") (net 5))
 (segment (start 124.5211 107.1968) (end 124.5211 113.1404) (width 0.3048) (layer "F.Cu") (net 5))
 (via (at 166.2787 113.1404) (size 0.7564) (drill 0.35) (layers "F.Cu" "B.Cu") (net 5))
 (via (at 162.0115 113.1404) (size 0.7564) (drill 0.35) (layers "F.Cu" "B.Cu") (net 5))
 (via (at 124.5211 113.1404) (size 0.7564) (drill 0.35) (layers "F.Cu" "B.Cu") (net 5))
 (via (at 112.0243 104.7584) (size 0.7564) (drill 0.35) (layers "F.Cu" "B.Cu") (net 5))
 (via (at 124.5211 107.1968) (size 0.7564) (drill 0.35) (layers "F.Cu" "B.Cu") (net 5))
 (segment (start 123.3019 107.1968) (end 124.5211 107.1968) (width 0.3048) (layer "B.Cu") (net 5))
 (segment (start 124.5211 113.1404) (end 133.2079 113.1404) (width 0.3048) (layer "B.Cu") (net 5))
 (segment (start 155.3059 116.798) (end 158.9635 113.1404) (width 0.3048) (layer "B.Cu") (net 5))
 (segment (start 158.9635 113.1404) (end 162.0115 113.1404) (width 0.3048) (layer "B.Cu") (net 5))
 (segment (start 101.2611 104.9036) (end 101.4063 104.7584) (width 0.3048) (layer "B.Cu") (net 5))
 (segment (start 171.2999 115.1136) (end 171.2999 116.8488) (width 0.3048) (layer "B.Cu") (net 5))
 (segment (start 136.8655 116.798) (end 155.3059 116.798) (width 0.3048) (layer "B.Cu") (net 5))
 (segment (start 124.5211 113.1404) (end 124.5211 116.7552) (width 0.3048) (layer "B.Cu") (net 5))
 (segment (start 133.2079 113.1404) (end 136.8655 116.798) (width 0.3048) (layer "B.Cu") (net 5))
 (segment (start 112.0243 104.7584) (end 120.8635 104.7584) (width 0.3048) (layer "B.Cu") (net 5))
 (segment (start 166.2787 113.1404) (end 169.3267 113.1404) (width 0.3048) (layer "B.Cu") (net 5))
 (segment (start 112.0243 104.7584) (end 101.4063 104.7584) (width 0.3048) (layer "B.Cu") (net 5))
 (segment (start 124.5211 116.7552) (end 124.5639 116.798) (width 0.3048) (layer "B.Cu") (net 5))
 (segment (start 123.3019 107.1968) (end 120.8635 104.7584) (width 0.3048) (layer "B.Cu") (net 5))
 (segment (start 169.3267 113.1404) (end 171.2999 115.1136) (width 0.3048) (layer "B.Cu") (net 5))
 (segment (start 110.1787 120.1712) (end 110.2111 120.2036) (width 1.27) (layer "F.Cu") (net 9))
 (segment (start 110.2111 120.2036) (end 110.4111 120.0036) (width 1.27) (layer "F.Cu") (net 9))
 (segment (start 101.3009 120.1712) (end 110.1787 120.1712) (width 1.27) (layer "F.Cu") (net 9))
 (via (at 110.4111 120.0036) (size 2.54) (drill 1.2) (layers "F.Cu" "B.Cu") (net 9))
 (segment (start 121.1683 119.2364) (end 165.0595 119.2364) (width 1.27) (layer "B.Cu") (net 9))
 (segment (start 101.2611 120.2036) (end 110.2111 120.2036) (width 1.27) (layer "B.Cu") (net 9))
 (segment (start 110.4111 120.0036) (end 112.8911 120.0036) (width 1.27) (layer "B.Cu") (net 9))
 (segment (start 166.2787 116.9076) (end 166.2199 116.8488) (width 1.27) (layer "B.Cu") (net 9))
 (segment (start 119.5915 120.8132) (end 121.1683 119.2364) (width 1.27) (layer "B.Cu") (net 9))
 (segment (start 112.8911 120.0036) (end 113.7007 120.8132) (width 1.27) (layer "B.Cu") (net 9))
 (segment (start 113.7007 120.8132) (end 119.5915 120.8132) (width 1.27) (layer "B.Cu") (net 9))
 (segment (start 110.4111 120.0036) (end 110.2821 120.1326) (width 1.27) (layer "B.Cu") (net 9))
 (segment (start 110.2111 120.2036) (end 110.4111 120.0036) (width 1.27) (layer "B.Cu") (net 9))
 (segment (start 166.2787 118.0172) (end 166.2787 116.9076) (width 1.27) (layer "B.Cu") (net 9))
 (segment (start 165.0595 119.2364) (end 166.2787 118.0172) (width 1.27) (layer "B.Cu") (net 9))
 (segment (start 101.2835 117.236) (end 105.9091 117.236) (width 1.27) (layer "F.Cu") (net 6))
 (segment (start 108.4111 117.2536) (end 105.9267 117.2536) (width 1.27) (layer "F.Cu") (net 6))
 (segment (start 105.9267 117.2536) (end 105.9283 117.2552) (width 1.27) (layer "F.Cu") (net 6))
 (segment (start 105.9267 117.2536) (end 105.9091 117.236) (width 1.27) (layer "F.Cu") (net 6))
 (via (at 108.4111 117.2536) (size 2.54) (drill 1.2) (layers "F.Cu" "B.Cu") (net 6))
 (segment (start 115.0723 119.2364) (end 113.0895 117.2536) (width 1.27) (layer "B.Cu") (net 6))
 (segment (start 108.3611 117.2036) (end 108.4111 117.2536) (width 1.27) (layer "B.Cu") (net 6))
 (segment (start 101.2611 117.2036) (end 108.3611 117.2036) (width 1.27) (layer "B.Cu") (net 6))
 (segment (start 113.0895 117.2536) (end 108.4111 117.2536) (width 1.27) (layer "B.Cu") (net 6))
 (segment (start 119.4839 117.8728) (end 119.4839 116.7472) (width 1.27) (layer "B.Cu") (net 6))
 (segment (start 118.1203 119.2364) (end 119.4839 117.8728) (width 1.27) (layer "B.Cu") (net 6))
 (segment (start 118.1203 119.2364) (end 115.0723 119.2364) (width 1.27) (layer "B.Cu") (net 6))
 (segment (start 107.7523 91.9616) (end 107.7571 91.9568) (width 1.27) (layer "F.Cu") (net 3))
 (segment (start 101.2263 91.9616) (end 107.7523 91.9616) (width 1.27) (layer "F.Cu") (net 3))
 (via (at 107.7571 91.9568) (size 1.3064) (drill 0.9) (layers "F.Cu" "B.Cu") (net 3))
 (segment (start 121.2883 94.5156) (end 118.7295 91.9568) (width 1.27) (layer "B.Cu") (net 3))
 (segment (start 195.8697 95.557) (end 194.8283 94.5156) (width 0.254) (layer "B.Cu") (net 3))
 (segment (start 192.6611 115.5036) (end 194.6611 113.5036) (width 0.254) (layer "B.Cu") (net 3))
 (segment (start 153.0199 110.702) (end 163.6719 110.702) (width 1.27) (layer "B.Cu") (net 3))
 (segment (start 107.7571 91.9568) (end 118.7295 91.9568) (width 1.27) (layer "B.Cu") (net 3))
 (segment (start 163.6799 116.8488) (end 163.6799 110.694) (width 1.27) (layer "B.Cu") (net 3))
 (segment (start 163.6719 110.702) (end 163.6799 110.694) (width 1.27) (layer "B.Cu") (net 3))
 (segment (start 194.6611 102.5036) (end 195.8697 101.295) (width 0.254) (layer "B.Cu") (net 3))
 (segment (start 121.2883 94.5156) (end 192.2883 94.5156) (width 1.27) (layer "B.Cu") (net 3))
 (segment (start 101.1911 92.0036) (end 101.2379 91.9568) (width 1.27) (layer "B.Cu") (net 3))
 (segment (start 116.9439 116.798) (end 116.9439 115.536) (width 1.27) (layer "B.Cu") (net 3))
 (segment (start 116.9439 115.536) (end 121.9303 110.5496) (width 1.27) (layer "B.Cu") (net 3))
 (segment (start 137.1703 107.9588) (end 150.2767 107.9588) (width 1.27) (layer "B.Cu") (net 3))
 (segment (start 101.2379 91.9568) (end 107.7571 91.9568) (width 1.27) (layer "B.Cu") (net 3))
 (segment (start 190.1971 115.5036) (end 192.6611 115.5036) (width 1.27) (layer "B.Cu") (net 3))
 (segment (start 192.2883 94.5156) (end 194.8283 94.5156) (width 1.27) (layer "B.Cu") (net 3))
 (segment (start 163.6799 110.694) (end 185.3875 110.694) (width 1.27) (layer "B.Cu") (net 3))
 (segment (start 195.8697 101.295) (end 195.8697 95.557) (width 0.254) (layer "B.Cu") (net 3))
 (segment (start 194.6611 113.5036) (end 194.6611 102.5036) (width 0.254) (layer "B.Cu") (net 3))
 (segment (start 185.3875 110.694) (end 190.1971 115.5036) (width 1.27) (layer "B.Cu") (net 3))
 (segment (start 134.5795 110.5496) (end 137.1703 107.9588) (width 1.27) (layer "B.Cu") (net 3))
 (segment (start 121.9303 110.5496) (end 134.5795 110.5496) (width 1.27) (layer "B.Cu") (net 3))
 (segment (start 150.2767 107.9588) (end 153.0199 110.702) (width 1.27) (layer "B.Cu") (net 3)))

